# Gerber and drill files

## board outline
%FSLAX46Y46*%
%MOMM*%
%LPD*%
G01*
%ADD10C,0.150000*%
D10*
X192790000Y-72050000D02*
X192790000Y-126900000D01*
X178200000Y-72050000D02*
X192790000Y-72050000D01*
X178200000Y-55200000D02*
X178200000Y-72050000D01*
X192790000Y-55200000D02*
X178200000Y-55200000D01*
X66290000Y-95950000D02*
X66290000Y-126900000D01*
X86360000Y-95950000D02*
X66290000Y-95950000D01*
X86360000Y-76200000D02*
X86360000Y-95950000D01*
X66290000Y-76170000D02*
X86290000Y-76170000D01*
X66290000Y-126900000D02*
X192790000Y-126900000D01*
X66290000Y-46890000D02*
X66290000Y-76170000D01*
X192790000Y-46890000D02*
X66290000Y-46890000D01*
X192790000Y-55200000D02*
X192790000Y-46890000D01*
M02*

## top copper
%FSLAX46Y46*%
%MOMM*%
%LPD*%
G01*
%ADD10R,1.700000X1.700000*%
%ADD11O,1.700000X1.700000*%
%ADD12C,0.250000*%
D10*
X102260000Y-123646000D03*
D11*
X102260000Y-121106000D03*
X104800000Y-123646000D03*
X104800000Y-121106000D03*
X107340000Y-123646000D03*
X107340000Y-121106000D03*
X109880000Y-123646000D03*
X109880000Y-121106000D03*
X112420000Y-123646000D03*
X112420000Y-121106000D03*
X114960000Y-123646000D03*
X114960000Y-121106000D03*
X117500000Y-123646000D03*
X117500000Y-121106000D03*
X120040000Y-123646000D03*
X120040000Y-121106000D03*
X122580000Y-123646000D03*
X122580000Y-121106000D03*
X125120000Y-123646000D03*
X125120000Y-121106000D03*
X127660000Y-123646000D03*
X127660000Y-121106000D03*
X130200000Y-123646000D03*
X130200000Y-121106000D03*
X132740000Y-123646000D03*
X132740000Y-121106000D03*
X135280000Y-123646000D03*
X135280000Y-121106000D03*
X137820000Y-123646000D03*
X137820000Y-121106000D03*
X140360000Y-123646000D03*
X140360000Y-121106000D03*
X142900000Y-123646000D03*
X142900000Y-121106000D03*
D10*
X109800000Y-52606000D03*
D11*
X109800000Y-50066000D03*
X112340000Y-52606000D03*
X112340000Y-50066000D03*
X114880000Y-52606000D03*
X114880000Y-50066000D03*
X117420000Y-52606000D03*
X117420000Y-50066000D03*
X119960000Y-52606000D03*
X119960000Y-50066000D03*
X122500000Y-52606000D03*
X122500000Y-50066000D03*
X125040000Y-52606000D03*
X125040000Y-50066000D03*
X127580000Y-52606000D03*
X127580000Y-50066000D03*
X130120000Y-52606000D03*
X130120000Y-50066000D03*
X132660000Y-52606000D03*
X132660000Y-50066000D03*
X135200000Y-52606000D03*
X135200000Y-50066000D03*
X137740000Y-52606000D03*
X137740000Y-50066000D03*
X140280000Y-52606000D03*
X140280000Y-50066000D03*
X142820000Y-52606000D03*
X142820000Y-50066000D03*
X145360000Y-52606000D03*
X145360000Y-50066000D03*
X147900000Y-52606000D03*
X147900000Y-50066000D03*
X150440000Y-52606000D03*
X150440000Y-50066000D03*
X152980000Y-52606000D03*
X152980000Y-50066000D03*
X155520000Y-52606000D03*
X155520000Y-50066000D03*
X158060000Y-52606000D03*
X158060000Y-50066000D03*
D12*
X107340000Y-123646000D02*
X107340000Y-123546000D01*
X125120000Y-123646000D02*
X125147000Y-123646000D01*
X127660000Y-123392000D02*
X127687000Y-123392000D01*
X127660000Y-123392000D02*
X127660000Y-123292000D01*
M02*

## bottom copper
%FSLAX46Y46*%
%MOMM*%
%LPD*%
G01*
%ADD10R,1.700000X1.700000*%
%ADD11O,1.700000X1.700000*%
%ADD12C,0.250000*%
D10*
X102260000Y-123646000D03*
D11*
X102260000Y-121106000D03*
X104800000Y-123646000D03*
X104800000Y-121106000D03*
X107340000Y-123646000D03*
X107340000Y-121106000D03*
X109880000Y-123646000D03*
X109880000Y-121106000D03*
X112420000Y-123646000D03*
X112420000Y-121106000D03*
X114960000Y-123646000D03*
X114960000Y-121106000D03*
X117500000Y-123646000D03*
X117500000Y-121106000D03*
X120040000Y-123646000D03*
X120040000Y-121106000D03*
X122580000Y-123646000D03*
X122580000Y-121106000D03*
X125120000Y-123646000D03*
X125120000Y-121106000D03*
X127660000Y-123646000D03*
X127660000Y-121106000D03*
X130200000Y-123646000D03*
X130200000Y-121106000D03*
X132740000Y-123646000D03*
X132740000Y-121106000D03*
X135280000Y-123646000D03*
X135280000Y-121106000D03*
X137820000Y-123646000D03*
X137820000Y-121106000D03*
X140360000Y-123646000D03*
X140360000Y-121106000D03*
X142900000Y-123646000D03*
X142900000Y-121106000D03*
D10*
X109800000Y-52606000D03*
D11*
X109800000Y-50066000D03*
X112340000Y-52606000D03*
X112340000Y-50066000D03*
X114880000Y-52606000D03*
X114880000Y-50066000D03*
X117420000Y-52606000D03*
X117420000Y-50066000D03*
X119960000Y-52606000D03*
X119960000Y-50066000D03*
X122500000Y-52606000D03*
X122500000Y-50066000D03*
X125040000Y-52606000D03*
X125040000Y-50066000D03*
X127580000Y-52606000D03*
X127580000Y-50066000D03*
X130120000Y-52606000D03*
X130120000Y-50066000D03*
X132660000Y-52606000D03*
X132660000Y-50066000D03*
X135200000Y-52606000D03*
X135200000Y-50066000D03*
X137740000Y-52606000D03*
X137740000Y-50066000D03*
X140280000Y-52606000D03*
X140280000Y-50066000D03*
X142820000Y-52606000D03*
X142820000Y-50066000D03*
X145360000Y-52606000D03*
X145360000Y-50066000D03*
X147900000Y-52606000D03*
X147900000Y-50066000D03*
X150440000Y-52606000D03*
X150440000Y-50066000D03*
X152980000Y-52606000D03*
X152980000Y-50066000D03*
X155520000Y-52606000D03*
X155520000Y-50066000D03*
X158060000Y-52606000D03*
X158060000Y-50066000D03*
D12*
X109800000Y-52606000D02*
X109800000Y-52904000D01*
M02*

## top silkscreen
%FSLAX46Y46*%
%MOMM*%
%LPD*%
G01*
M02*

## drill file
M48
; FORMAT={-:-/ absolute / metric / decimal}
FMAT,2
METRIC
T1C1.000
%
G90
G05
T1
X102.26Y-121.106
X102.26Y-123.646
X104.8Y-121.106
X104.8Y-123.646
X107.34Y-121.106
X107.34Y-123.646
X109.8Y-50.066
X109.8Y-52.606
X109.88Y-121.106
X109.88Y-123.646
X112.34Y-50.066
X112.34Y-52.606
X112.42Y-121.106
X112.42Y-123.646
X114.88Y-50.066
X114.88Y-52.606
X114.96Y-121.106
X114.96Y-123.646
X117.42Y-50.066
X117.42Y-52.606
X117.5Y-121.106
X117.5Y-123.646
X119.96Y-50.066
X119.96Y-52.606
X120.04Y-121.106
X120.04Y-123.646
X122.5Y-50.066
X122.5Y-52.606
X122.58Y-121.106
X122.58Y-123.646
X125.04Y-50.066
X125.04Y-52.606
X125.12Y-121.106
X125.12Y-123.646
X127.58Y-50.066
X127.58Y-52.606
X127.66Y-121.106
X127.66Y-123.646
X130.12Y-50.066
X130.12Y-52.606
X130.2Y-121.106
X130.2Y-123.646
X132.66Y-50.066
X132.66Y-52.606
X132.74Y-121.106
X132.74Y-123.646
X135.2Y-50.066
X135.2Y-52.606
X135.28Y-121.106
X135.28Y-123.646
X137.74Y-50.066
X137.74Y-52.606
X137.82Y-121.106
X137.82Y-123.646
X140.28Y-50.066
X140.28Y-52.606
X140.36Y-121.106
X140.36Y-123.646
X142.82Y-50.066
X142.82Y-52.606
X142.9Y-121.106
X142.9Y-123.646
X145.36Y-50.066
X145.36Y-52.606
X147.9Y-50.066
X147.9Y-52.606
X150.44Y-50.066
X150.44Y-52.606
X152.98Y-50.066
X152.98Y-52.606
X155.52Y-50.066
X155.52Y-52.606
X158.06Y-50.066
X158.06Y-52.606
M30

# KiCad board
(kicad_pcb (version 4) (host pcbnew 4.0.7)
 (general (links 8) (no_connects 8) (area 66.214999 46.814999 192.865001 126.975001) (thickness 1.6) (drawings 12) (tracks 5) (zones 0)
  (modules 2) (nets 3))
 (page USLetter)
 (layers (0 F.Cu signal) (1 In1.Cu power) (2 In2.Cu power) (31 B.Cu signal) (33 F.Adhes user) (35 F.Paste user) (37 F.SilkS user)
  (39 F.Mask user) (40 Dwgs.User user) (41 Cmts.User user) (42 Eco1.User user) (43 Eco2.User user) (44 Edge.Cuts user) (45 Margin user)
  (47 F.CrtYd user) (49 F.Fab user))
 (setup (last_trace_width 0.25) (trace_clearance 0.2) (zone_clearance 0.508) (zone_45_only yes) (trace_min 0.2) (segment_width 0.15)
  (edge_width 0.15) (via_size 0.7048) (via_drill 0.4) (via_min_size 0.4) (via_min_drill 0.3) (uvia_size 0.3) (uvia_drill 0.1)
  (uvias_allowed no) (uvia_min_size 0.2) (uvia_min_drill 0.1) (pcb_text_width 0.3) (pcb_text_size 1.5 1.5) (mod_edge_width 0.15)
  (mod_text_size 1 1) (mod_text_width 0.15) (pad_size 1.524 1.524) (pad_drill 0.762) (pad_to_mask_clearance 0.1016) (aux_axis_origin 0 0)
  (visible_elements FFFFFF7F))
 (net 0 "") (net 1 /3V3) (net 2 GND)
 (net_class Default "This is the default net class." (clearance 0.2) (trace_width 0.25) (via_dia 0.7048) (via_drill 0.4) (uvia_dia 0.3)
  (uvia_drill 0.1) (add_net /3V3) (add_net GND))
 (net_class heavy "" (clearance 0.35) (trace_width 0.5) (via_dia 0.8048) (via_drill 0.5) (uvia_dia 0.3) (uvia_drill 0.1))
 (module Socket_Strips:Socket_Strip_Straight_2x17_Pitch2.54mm (layer B.Cu) (at 102.26 123.646 270)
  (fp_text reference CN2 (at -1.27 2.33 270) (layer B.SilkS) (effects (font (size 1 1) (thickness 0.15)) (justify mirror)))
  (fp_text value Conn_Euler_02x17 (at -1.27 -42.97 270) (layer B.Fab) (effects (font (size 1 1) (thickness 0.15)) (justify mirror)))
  (pad 1 thru_hole rect (at 0 0 270) (size 1.7 1.7) (drill 1) (layers *.Cu *.Mask) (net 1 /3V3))
  (pad 2 thru_hole oval (at -2.54 0 270) (size 1.7 1.7) (drill 1) (layers *.Cu *.Mask))
  (pad 3 thru_hole oval (at 0 -2.54 270) (size 1.7 1.7) (drill 1) (layers *.Cu *.Mask))
  (pad 4 thru_hole oval (at -2.54 -2.54 270) (size 1.7 1.7) (drill 1) (layers *.Cu *.Mask))
  (pad 5 thru_hole oval (at 0 -5.08 270) (size 1.7 1.7) (drill 1) (layers *.Cu *.Mask))
  (pad 6 thru_hole oval (at -2.54 -5.08 270) (size 1.7 1.7) (drill 1) (layers *.Cu *.Mask) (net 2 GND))
  (pad 7 thru_hole oval (at 0 -7.62 270) (size 1.7 1.7) (drill 1) (layers *.Cu *.Mask))
  (pad 8 thru_hole oval (at -2.54 -7.62 270) (size 1.7 1.7) (drill 1) (layers *.Cu *.Mask))
  (pad 9 thru_hole oval (at 0 -10.16 270) (size 1.7 1.7) (drill 1) (layers *.Cu *.Mask) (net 2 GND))
  (pad 10 thru_hole oval (at -2.54 -10.16 270) (size 1.7 1.7) (drill 1) (layers *.Cu *.Mask))
  (pad 11 thru_hole oval (at 0 -12.7 270) (size 1.7 1.7) (drill 1) (layers *.Cu *.Mask))
  (pad 12 thru_hole oval (at -2.54 -12.7 270) (size 1.7 1.7) (drill 1) (layers *.Cu *.Mask))
  (pad 13 thru_hole oval (at 0 -15.24 270) (size 1.7 1.7) (drill 1) (layers *.Cu *.Mask))
  (pad 14 thru_hole oval (at -2.54 -15.24 270) (size 1.7 1.7) (drill 1) (layers *.Cu *.Mask))
  (pad 15 thru_hole oval (at 0 -17.78 270) (size 1.7 1.7) (drill 1) (layers *.Cu *.Mask))
  (pad 16 thru_hole oval (at -2.54 -17.78 270) (size 1.7 1.7) (drill 1) (layers *.Cu *.Mask))
  (pad 17 thru_hole oval (at 0 -20.32 270) (size 1.7 1.7) (drill 1) (layers *.Cu *.Mask) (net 1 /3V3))
  (pad 18 thru_hole oval (at -2.54 -20.32 270) (size 1.7 1.7) (drill 1) (layers *.Cu *.Mask))
  (pad 19 thru_hole oval (at 0 -22.86 270) (size 1.7 1.7) (drill 1) (layers *.Cu *.Mask))
  (pad 20 thru_hole oval (at -2.54 -22.86 270) (size 1.7 1.7) (drill 1) (layers *.Cu *.Mask))
  (pad 21 thru_hole oval (at 0 -25.4 270) (size 1.7 1.7) (drill 1) (layers *.Cu *.Mask))
  (pad 22 thru_hole oval (at -2.54 -25.4 270) (size 1.7 1.7) (drill 1) (layers *.Cu *.Mask))
  (pad 23 thru_hole oval (at 0 -27.94 270) (size 1.7 1.7) (drill 1) (layers *.Cu *.Mask))
  (pad 24 thru_hole oval (at -2.54 -27.94 270) (size 1.7 1.7) (drill 1) (layers *.Cu *.Mask))
  (pad 25 thru_hole oval (at 0 -30.48 270) (size 1.7 1.7) (drill 1) (layers *.Cu *.Mask) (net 2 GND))
  (pad 26 thru_hole oval (at -2.54 -30.48 270) (size 1.7 1.7) (drill 1) (layers *.Cu *.Mask))
  (pad 27 thru_hole oval (at 0 -33.02 270) (size 1.7 1.7) (drill 1) (layers *.Cu *.Mask))
  (pad 28 thru_hole oval (at -2.54 -33.02 270) (size 1.7 1.7) (drill 1) (layers *.Cu *.Mask))
  (pad 29 thru_hole oval (at 0 -35.56 270) (size 1.7 1.7) (drill 1) (layers *.Cu *.Mask))
  (pad 30 thru_hole oval (at -2.54 -35.56 270) (size 1.7 1.7) (drill 1) (layers *.Cu *.Mask))
  (pad 31 thru_hole oval (at 0 -38.1 270) (size 1.7 1.7) (drill 1) (layers *.Cu *.Mask))
  (pad 32 thru_hole oval (at -2.54 -38.1 270) (size 1.7 1.7) (drill 1) (layers *.Cu *.Mask))
  (pad 33 thru_hole oval (at 0 -40.64 270) (size 1.7 1.7) (drill 1) (layers *.Cu *.Mask))
  (pad 34 thru_hole oval (at -2.54 -40.64 270) (size 1.7 1.7) (drill 1) (layers *.Cu *.Mask)))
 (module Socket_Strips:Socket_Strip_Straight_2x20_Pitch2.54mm (layer B.Cu) (at 109.8 52.606 270)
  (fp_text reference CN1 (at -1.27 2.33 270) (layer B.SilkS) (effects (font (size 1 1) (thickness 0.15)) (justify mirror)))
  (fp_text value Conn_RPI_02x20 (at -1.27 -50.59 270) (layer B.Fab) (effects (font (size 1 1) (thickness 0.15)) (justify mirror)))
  (pad 1 thru_hole rect (at 0 0 270) (size 1.7 1.7) (drill 1) (layers *.Cu *.Mask) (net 1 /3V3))
  (pad 2 thru_hole oval (at -2.54 0 270) (size 1.7 1.7) (drill 1) (layers *.Cu *.Mask))
  (pad 3 thru_hole oval (at 0 -2.54 270) (size 1.7 1.7) (drill 1) (layers *.Cu *.Mask))
  (pad 4 thru_hole oval (at -2.54 -2.54 270) (size 1.7 1.7) (drill 1) (layers *.Cu *.Mask))
  (pad 5 thru_hole oval (at 0 -5.08 270) (size 1.7 1.7) (drill 1) (layers *.Cu *.Mask))
  (pad 6 thru_hole oval (at -2.54 -5.08 270) (size 1.7 1.7) (drill 1) (layers *.Cu *.Mask))
  (pad 7 thru_hole oval (at 0 -7.62 270) (size 1.7 1.7) (drill 1) (layers *.Cu *.Mask))
  (pad 8 thru_hole oval (at -2.54 -7.62 270) (size 1.7 1.7) (drill 1) (layers *.Cu *.Mask))
  (pad 9 thru_hole oval (at 0 -10.16 270) (size 1.7 1.7) (drill 1) (layers *.Cu *.Mask) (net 2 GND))
  (pad 10 thru_hole oval (at -2.54 -10.16 270) (size 1.7 1.7) (drill 1) (layers *.Cu *.Mask))
  (pad 11 thru_hole oval (at 0 -12.7 270) (size 1.7 1.7) (drill 1) (layers *.Cu *.Mask))
  (pad 12 thru_hole oval (at -2.54 -12.7 270) (size 1.7 1.7) (drill 1) (layers *.Cu *.Mask))
  (pad 13 thru_hole oval (at 0 -15.24 270) (size 1.7 1.7) (drill 1) (layers *.Cu *.Mask))
  (pad 14 thru_hole oval (at -2.54 -15.24 270) (size 1.7 1.7) (drill 1) (layers *.Cu *.Mask) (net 2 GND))
  (pad 15 thru_hole oval (at 0 -17.78 270) (size 1.7 1.7) (drill 1) (layers *.Cu *.Mask))
  (pad 16 thru_hole oval (at -2.54 -17.78 270) (size 1.7 1.7) (drill 1) (layers *.Cu *.Mask))
  (pad 17 thru_hole oval (at 0 -20.32 270) (size 1.7 1.7) (drill 1) (layers *.Cu *.Mask) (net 1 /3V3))
  (pad 18 thru_hole oval (at -2.54 -20.32 270) (size 1.7 1.7) (drill 1) (layers *.Cu *.Mask))
  (pad 19 thru_hole oval (at 0 -22.86 270) (size 1.7 1.7) (drill 1) (layers *.Cu *.Mask))
  (pad 20 thru_hole oval (at -2.54 -22.86 270) (size 1.7 1.7) (drill 1) (layers *.Cu *.Mask))
  (pad 21 thru_hole oval (at 0 -25.4 270) (size 1.7 1.7) (drill 1) (layers *.Cu *.Mask))
  (pad 22 thru_hole oval (at -2.54 -25.4 270) (size 1.7 1.7) (drill 1) (layers *.Cu *.Mask))
  (pad 23 thru_hole oval (at 0 -27.94 270) (size 1.7 1.7) (drill 1) (layers *.Cu *.Mask))
  (pad 24 thru_hole oval (at -2.54 -27.94 270) (size 1.7 1.7) (drill 1) (layers *.Cu *.Mask))
  (pad 25 thru_hole oval (at 0 -30.48 270) (size 1.7 1.7) (drill 1) (layers *.Cu *.Mask) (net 2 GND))
  (pad 26 thru_hole oval (at -2.54 -30.48 270) (size 1.7 1.7) (drill 1) (layers *.Cu *.Mask))
  (pad 27 thru_hole oval (at 0 -33.02 270) (size 1.7 1.7) (drill 1) (layers *.Cu *.Mask))
  (pad 28 thru_hole oval (at -2.54 -33.02 270) (size 1.7 1.7) (drill 1) (layers *.Cu *.Mask))
  (pad 29 thru_hole oval (at 0 -35.56 270) (size 1.7 1.7) (drill 1) (layers *.Cu *.Mask))
  (pad 30 thru_hole oval (at -2.54 -35.56 270) (size 1.7 1.7) (drill 1) (layers *.Cu *.Mask))
  (pad 31 thru_hole oval (at 0 -38.1 270) (size 1.7 1.7) (drill 1) (layers *.Cu *.Mask))
  (pad 32 thru_hole oval (at -2.54 -38.1 270) (size 1.7 1.7) (drill 1) (layers *.Cu *.Mask))
  (pad 33 thru_hole oval (at 0 -40.64 270) (size 1.7 1.7) (drill 1) (layers *.Cu *.Mask))
  (pad 34 thru_hole oval (at -2.54 -40.64 270) (size 1.7 1.7) (drill 1) (layers *.Cu *.Mask))
  (pad 35 thru_hole oval (at 0 -43.18 270) (size 1.7 1.7) (drill 1) (layers *.Cu *.Mask))
  (pad 36 thru_hole oval (at -2.54 -43.18 270) (size 1.7 1.7) (drill 1) (layers *.Cu *.Mask))
  (pad 37 thru_hole oval (at 0 -45.72 270) (size 1.7 1.7) (drill 1) (layers *.Cu *.Mask))
  (pad 38 thru_hole oval (at -2.54 -45.72 270) (size 1.7 1.7) (drill 1) (layers *.Cu *.Mask))
  (pad 39 thru_hole oval (at 0 -48.26 270) (size 1.7 1.7) (drill 1) (layers *.Cu *.Mask))
  (pad 40 thru_hole oval (at -2.54 -48.26 270) (size 1.7 1.7) (drill 1) (layers *.Cu *.Mask)))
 (gr_line (start 192.79 72.05) (end 192.79 126.9) (angle 90) (layer Edge.Cuts) (width 0.15))
 (gr_line (start 178.2 72.05) (end 192.79 72.05) (angle 90) (layer Edge.Cuts) (width 0.15))
 (gr_line (start 178.2 55.2) (end 178.2 72.05) (angle 90) (layer Edge.Cuts) (width 0.15))
 (gr_line (start 192.79 55.2) (end 178.2 55.2) (angle 90) (layer Edge.Cuts) (width 0.15))
 (gr_line (start 66.29 95.95) (end 66.29 126.9) (angle 90) (layer Edge.Cuts) (width 0.15))
 (gr_line (start 86.36 95.95) (end 66.29 95.95) (angle 90) (layer Edge.Cuts) (width 0.15))
 (gr_line (start 86.36 76.2) (end 86.36 95.95) (angle 90) (layer Edge.Cuts) (width 0.15))
 (gr_line (start 66.29 76.17) (end 86.29 76.17) (angle 90) (layer Edge.Cuts) (width 0.15))
 (gr_line (start 66.29 126.9) (end 192.79 126.9) (angle 90) (layer Edge.Cuts) (width 0.15))
 (gr_line (start 66.29 46.89) (end 66.29 76.17) (angle 90) (layer Edge.Cuts) (width 0.15))
 (gr_line (start 192.79 46.89) (end 66.29 46.89) (angle 90) (layer Edge.Cuts) (width 0.15))
 (gr_line (start 192.79 55.2) (end 192.79 46.89) (angle 90) (layer Edge.Cuts) (width 0.15))
 (segment (start 107.34 123.646) (end 107.34 123.546) (width 0.25) (layer F.Cu) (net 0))
 (segment (start 125.12 123.646) (end 125.147 123.646) (width 0.25) (layer F.Cu) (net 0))
 (segment (start 127.66 123.392) (end 127.687 123.392) (width 0.25) (layer F.Cu) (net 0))
 (segment (start 127.66 123.392) (end 127.66 123.292) (width 0.25) (layer F.Cu) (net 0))
 (segment (start 109.8 52.606) (end 109.8 52.904) (width 0.25) (layer B.Cu) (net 1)))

